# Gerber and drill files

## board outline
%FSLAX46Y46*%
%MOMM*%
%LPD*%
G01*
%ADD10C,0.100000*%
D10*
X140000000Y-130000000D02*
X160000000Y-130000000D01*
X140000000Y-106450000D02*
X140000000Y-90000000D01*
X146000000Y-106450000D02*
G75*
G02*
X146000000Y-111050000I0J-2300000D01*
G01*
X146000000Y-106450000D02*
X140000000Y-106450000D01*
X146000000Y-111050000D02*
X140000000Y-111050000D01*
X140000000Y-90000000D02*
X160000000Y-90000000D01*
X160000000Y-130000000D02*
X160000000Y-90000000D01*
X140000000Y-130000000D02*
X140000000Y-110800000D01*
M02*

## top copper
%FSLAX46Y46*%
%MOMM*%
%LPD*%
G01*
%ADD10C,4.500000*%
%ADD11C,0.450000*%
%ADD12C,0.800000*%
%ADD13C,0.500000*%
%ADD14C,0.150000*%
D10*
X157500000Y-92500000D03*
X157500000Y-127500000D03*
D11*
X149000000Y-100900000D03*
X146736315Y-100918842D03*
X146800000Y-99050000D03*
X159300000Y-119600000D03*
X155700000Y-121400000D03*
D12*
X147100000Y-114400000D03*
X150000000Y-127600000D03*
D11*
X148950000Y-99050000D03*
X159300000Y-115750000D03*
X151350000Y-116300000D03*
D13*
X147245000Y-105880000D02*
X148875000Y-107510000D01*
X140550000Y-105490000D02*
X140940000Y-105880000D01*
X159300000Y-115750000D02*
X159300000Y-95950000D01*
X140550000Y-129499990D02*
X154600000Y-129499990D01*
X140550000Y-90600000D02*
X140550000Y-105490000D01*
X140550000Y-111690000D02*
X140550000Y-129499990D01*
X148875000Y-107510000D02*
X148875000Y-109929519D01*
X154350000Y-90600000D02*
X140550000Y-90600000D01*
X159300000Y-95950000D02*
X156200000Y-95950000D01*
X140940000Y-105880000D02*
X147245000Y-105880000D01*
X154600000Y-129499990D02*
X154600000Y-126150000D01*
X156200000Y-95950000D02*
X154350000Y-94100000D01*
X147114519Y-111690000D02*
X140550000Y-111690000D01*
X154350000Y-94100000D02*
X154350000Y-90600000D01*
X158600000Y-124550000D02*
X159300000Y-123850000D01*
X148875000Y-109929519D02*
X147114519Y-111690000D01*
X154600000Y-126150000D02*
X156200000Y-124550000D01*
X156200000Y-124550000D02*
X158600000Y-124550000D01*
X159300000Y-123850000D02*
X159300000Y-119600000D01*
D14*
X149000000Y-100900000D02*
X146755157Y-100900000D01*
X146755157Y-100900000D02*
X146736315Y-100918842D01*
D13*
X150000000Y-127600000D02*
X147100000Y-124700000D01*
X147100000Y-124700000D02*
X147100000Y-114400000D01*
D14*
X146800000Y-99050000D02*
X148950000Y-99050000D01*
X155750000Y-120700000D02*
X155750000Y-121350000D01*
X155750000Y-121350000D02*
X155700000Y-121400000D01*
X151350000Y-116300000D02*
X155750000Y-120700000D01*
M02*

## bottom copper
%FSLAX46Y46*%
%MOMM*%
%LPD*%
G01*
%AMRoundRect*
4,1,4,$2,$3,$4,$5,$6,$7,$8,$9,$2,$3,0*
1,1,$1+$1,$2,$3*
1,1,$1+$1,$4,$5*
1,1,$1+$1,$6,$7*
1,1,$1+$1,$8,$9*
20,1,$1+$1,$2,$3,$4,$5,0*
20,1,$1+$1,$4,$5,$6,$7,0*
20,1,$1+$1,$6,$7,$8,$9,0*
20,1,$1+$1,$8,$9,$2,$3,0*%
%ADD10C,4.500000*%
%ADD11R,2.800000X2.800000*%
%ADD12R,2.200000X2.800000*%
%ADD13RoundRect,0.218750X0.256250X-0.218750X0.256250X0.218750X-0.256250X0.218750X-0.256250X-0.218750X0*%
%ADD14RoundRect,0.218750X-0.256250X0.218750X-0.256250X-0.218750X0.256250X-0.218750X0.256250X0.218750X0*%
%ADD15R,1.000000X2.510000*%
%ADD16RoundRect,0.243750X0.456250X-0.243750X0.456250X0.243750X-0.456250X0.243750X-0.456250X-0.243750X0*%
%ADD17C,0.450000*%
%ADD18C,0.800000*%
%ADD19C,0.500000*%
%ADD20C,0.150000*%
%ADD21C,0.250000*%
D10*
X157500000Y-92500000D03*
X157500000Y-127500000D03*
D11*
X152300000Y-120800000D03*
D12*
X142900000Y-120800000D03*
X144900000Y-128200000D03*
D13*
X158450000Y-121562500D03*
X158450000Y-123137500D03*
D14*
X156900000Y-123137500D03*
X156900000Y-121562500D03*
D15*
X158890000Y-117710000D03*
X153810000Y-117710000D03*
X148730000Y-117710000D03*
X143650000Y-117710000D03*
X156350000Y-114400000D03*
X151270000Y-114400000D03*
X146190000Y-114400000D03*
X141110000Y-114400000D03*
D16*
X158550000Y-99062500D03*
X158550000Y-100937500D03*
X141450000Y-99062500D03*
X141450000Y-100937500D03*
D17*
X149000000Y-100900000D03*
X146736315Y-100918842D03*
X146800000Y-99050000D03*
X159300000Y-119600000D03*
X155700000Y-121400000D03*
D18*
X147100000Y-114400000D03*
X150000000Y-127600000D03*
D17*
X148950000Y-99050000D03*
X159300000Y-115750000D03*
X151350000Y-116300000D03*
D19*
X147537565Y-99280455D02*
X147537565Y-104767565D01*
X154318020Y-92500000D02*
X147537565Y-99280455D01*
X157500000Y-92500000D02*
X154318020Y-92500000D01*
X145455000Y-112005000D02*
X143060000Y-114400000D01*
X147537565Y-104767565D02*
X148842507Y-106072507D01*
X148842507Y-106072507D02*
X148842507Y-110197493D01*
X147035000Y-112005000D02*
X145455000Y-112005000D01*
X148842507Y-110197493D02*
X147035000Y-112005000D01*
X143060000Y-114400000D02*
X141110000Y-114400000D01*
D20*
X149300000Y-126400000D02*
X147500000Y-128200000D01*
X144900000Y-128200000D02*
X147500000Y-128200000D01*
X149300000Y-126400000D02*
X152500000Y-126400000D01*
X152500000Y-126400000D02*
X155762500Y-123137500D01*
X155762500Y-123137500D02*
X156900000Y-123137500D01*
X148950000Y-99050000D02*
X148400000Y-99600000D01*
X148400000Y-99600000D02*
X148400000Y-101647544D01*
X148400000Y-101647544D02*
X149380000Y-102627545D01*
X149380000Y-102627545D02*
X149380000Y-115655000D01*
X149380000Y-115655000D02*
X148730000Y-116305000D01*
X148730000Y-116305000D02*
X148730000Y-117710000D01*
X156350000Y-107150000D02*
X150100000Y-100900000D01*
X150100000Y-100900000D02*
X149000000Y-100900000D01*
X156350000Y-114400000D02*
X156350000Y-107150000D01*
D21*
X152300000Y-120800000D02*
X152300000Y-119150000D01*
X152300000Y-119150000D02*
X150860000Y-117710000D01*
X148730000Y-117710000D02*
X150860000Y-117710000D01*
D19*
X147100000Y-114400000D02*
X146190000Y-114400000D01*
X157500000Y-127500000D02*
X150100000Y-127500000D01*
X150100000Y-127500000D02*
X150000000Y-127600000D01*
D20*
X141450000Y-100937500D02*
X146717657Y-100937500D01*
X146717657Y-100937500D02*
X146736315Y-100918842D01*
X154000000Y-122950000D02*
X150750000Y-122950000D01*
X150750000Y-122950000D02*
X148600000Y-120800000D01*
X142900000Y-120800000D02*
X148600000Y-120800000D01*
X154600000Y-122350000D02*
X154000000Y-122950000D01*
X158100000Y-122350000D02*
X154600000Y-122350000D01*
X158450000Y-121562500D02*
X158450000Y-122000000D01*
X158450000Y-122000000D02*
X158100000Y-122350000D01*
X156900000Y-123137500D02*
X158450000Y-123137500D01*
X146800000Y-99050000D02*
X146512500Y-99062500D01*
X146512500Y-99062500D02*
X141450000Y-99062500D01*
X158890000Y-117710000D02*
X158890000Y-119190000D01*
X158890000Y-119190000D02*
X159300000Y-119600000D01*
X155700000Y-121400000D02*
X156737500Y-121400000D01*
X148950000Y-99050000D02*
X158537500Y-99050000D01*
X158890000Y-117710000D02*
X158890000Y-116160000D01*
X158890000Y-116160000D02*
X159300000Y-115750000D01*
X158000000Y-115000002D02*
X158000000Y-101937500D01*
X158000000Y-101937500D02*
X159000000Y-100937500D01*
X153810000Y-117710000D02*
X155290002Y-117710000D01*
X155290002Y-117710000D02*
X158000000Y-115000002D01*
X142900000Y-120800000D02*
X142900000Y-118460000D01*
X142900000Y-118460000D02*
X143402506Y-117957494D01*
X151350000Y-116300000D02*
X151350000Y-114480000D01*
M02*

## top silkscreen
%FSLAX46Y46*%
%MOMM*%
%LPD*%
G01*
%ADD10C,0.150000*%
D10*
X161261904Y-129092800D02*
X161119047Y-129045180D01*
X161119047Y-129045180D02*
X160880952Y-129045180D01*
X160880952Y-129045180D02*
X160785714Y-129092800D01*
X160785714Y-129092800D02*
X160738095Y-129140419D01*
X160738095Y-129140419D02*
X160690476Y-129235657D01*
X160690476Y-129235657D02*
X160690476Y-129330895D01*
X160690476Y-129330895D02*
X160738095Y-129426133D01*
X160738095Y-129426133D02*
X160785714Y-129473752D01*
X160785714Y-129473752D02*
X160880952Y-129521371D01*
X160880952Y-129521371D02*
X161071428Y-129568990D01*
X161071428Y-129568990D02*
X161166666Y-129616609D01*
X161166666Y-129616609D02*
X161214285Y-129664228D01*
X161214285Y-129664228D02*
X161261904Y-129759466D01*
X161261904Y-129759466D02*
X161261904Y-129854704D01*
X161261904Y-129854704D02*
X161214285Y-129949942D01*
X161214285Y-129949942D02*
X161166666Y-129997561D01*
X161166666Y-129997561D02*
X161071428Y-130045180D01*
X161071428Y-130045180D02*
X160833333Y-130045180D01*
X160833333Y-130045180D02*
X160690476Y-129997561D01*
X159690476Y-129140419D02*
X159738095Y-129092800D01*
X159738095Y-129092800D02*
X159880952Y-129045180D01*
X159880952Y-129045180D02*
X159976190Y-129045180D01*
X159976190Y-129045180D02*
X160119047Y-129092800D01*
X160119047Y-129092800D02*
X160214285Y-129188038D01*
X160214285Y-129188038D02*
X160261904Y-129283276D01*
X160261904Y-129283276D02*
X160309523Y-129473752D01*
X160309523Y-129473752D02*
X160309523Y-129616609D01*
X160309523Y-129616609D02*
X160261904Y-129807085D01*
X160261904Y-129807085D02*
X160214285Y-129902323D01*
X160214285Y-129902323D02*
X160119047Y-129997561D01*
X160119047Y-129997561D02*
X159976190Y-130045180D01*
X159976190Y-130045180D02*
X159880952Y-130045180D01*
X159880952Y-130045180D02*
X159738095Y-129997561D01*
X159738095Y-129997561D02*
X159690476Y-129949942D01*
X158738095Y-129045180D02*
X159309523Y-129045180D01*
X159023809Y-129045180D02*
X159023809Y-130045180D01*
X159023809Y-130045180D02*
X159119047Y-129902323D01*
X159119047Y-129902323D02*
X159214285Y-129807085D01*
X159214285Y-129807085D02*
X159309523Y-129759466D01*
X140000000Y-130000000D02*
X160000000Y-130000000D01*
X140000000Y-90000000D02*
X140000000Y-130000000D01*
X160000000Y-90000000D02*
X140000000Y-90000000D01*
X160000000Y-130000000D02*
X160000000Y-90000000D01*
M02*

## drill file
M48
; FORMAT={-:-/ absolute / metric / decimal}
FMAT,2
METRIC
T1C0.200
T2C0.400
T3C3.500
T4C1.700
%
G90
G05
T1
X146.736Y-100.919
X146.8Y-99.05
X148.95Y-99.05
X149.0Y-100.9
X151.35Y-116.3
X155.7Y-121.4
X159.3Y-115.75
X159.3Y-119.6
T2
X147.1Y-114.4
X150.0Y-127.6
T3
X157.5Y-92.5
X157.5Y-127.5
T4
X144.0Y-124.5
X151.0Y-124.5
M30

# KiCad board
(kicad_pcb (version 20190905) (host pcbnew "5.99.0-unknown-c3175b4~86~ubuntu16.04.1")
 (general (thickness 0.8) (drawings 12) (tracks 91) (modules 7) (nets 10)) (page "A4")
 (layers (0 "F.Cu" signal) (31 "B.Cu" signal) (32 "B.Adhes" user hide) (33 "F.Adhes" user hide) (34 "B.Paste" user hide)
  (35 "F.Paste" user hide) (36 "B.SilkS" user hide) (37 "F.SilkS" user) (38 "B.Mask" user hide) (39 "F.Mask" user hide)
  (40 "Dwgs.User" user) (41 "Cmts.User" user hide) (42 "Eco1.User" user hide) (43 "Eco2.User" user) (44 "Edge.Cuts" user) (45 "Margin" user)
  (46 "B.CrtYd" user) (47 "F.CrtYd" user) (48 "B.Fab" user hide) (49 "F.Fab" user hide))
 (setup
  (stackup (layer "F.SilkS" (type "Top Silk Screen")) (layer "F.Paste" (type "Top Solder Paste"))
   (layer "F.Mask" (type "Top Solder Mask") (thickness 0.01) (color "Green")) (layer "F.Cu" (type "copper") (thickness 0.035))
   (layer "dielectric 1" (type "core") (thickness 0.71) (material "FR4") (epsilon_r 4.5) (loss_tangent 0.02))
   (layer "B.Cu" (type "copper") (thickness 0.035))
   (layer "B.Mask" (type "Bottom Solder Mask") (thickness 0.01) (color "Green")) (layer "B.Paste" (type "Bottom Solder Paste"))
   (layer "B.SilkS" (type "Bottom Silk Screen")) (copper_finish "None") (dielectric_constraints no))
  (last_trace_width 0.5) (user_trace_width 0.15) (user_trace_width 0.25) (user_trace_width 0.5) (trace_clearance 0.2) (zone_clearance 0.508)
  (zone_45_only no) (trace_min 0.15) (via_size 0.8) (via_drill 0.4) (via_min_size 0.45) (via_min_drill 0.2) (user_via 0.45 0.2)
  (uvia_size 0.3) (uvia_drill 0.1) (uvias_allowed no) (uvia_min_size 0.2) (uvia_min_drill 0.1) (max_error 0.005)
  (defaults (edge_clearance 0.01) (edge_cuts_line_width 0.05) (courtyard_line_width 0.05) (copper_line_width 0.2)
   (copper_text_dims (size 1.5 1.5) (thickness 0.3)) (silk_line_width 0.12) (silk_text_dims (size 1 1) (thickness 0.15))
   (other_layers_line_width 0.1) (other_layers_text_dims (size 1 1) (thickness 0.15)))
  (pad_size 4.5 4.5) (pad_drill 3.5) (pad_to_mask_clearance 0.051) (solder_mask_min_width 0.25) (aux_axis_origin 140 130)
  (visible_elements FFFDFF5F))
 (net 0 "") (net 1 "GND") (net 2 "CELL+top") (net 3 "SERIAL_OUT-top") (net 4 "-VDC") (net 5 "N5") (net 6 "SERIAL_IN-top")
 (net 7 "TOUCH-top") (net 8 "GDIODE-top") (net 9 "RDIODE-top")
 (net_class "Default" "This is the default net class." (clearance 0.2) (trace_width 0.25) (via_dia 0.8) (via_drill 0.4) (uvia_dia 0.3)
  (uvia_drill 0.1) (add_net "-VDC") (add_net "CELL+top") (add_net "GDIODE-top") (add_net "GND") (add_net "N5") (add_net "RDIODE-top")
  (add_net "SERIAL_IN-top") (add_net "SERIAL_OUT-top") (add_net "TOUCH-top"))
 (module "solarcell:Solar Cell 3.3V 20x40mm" (layer "F.Cu") (at 160 130 180)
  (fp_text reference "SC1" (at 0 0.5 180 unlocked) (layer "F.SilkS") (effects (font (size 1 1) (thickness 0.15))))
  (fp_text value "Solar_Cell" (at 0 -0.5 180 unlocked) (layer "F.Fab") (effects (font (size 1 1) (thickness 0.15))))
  (fp_line (start 20 0) (end 0 0) (layer "F.SilkS") (width 0.15))
  (fp_line (start 20 40) (end 20 0) (layer "F.SilkS") (width 0.15))
  (fp_line (start 0 40) (end 20 40) (layer "F.SilkS") (width 0.15))
  (fp_line (start 0 0) (end 0 40) (layer "F.SilkS") (width 0.15))
  (pad "2" thru_hole circle (at 2.5 37.5 180) (size 4.5 4.5) (drill 3.5) (layers *.Cu *.Mask) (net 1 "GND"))
  (pad "1" thru_hole circle (at 2.5 2.5 180) (size 4.5 4.5) (drill 3.5) (layers *.Cu *.Mask) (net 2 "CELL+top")))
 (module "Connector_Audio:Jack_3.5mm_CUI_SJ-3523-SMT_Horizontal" (layer "B.Cu") (at 146.5 124.5 -90)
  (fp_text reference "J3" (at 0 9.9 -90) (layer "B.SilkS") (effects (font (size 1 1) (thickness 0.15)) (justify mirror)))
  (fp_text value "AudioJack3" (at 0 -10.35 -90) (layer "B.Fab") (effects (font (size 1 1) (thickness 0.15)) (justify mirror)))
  (pad "" np_thru_hole circle (at 0 -4.5 270) (size 1.7 1.7) (drill 1.7) (layers *.Cu *.Mask))
  (pad "" np_thru_hole circle (at 0 2.5 270) (size 1.7 1.7) (drill 1.7) (layers *.Cu *.Mask))
  (pad "T" smd rect (at -3.7 -5.8 270) (size 2.8 2.8) (layers "B.Cu" "B.Paste" "B.Mask") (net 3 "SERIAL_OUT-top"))
  (pad "S" smd rect (at -3.7 3.6 270) (size 2.8 2.2) (layers "B.Cu" "B.Paste" "B.Mask") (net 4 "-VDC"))
  (pad "R" smd rect (at 3.7 1.6 270) (size 2.8 2.2) (layers "B.Cu" "B.Paste" "B.Mask") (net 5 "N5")))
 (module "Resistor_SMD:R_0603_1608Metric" (layer "B.Cu") (at 158.45 122.35 90)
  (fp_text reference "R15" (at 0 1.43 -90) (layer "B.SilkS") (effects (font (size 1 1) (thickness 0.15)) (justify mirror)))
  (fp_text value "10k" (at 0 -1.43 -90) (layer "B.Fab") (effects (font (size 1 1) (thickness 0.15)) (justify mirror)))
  (pad "2" smd roundrect (at 0.7875 0 90) (size 0.875 0.95) (layers "B.Cu" "B.Paste" "B.Mask") (roundrect_rratio 0.25) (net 4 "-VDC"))
  (pad "1" smd roundrect (at -0.7875 0 90) (size 0.875 0.95) (layers "B.Cu" "B.Paste" "B.Mask") (roundrect_rratio 0.25) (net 5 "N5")))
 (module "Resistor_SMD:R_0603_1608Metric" (layer "B.Cu") (at 156.9 122.35 -90)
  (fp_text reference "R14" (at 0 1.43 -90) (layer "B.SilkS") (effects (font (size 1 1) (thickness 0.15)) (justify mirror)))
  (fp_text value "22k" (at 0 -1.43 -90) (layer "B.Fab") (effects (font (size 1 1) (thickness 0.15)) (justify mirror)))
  (pad "2" smd roundrect (at 0.7875 0 270) (size 0.875 0.95) (layers "B.Cu" "B.Paste" "B.Mask") (roundrect_rratio 0.25) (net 5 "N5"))
  (pad "1" smd roundrect (at -0.7875 0 270) (size 0.875 0.95) (layers "B.Cu" "B.Paste" "B.Mask") (roundrect_rratio 0.25)
   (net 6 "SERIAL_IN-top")))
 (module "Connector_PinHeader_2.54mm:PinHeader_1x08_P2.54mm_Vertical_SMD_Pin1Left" (layer "B.Cu") (at 150 116.055 -90)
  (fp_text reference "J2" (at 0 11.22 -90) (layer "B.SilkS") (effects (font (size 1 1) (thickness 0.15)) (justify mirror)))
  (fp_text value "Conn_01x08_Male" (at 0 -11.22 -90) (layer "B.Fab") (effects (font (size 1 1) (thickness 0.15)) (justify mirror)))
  (pad "8" smd rect (at 1.655 -8.89 270) (size 2.51 1) (layers "B.Cu" "B.Paste" "B.Mask") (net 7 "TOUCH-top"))
  (pad "6" smd rect (at 1.655 -3.81 270) (size 2.51 1) (layers "B.Cu" "B.Paste" "B.Mask") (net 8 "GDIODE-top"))
  (pad "4" smd rect (at 1.655 1.27 270) (size 2.51 1) (layers "B.Cu" "B.Paste" "B.Mask") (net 3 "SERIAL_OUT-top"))
  (pad "2" smd rect (at 1.655 6.35 270) (size 2.51 1) (layers "B.Cu" "B.Paste" "B.Mask") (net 4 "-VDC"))
  (pad "7" smd rect (at -1.655 -6.35 270) (size 2.51 1) (layers "B.Cu" "B.Paste" "B.Mask") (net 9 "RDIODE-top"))
  (pad "5" smd rect (at -1.655 -1.27 270) (size 2.51 1) (layers "B.Cu" "B.Paste" "B.Mask") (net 6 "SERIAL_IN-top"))
  (pad "3" smd rect (at -1.655 3.81 270) (size 2.51 1) (layers "B.Cu" "B.Paste" "B.Mask") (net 2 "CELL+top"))
  (pad "1" smd rect (at -1.655 8.89 270) (size 2.51 1) (layers "B.Cu" "B.Paste" "B.Mask") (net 1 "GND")))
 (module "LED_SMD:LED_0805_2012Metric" (layer "B.Cu") (at 158.55 100 90)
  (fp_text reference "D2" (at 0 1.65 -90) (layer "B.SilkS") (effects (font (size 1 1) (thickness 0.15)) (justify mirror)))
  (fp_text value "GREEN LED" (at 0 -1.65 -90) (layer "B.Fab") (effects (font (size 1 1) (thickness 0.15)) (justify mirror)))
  (pad "2" smd roundrect (at 0.9375 0 90) (size 0.975 1.4) (layers "B.Cu" "B.Paste" "B.Mask") (roundrect_rratio 0.25)
   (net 3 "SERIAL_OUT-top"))
  (pad "1" smd roundrect (at -0.9375 0 90) (size 0.975 1.4) (layers "B.Cu" "B.Paste" "B.Mask") (roundrect_rratio 0.25) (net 8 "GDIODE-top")))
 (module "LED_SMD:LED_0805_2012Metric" (layer "B.Cu") (at 141.45 100 90)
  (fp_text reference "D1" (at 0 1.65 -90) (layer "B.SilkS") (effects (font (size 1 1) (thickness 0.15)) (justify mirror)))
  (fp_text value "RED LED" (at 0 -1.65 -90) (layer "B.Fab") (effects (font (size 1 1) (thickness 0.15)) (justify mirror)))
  (pad "2" smd roundrect (at 0.9375 0 90) (size 0.975 1.4) (layers "B.Cu" "B.Paste" "B.Mask") (roundrect_rratio 0.25)
   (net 3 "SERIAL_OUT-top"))
  (pad "1" smd roundrect (at -0.9375 0 90) (size 0.975 1.4) (layers "B.Cu" "B.Paste" "B.Mask") (roundrect_rratio 0.25) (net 9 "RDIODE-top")))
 (gr_line (start 140 130) (end 160 130) (layer "Edge.Cuts") (width 0.1))
 (gr_line (start 140 106.45) (end 140 90) (layer "Edge.Cuts") (width 0.1))
 (gr_arc (start 146 108.75) (end 146 106.45) (angle 180) (layer "Edge.Cuts") (width 0.1))
 (gr_line (start 146 106.45) (end 140 106.45) (layer "Edge.Cuts") (width 0.1))
 (gr_line (start 146 111.05) (end 140 111.05) (layer "Edge.Cuts") (width 0.1))
 (gr_line (start 140 90) (end 160 90) (layer "Edge.Cuts") (width 0.1))
 (gr_line (start 160 130) (end 160 90) (layer "Edge.Cuts") (width 0.1))
 (gr_line (start 140 130) (end 140 110.8) (layer "Edge.Cuts") (width 0.1))
 (segment (start 147.537565 99.280455) (end 147.537565 104.767565) (width 0.5) (layer "B.Cu") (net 1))
 (segment (start 154.31802 92.5) (end 147.537565 99.280455) (width 0.5) (layer "B.Cu") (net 1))
 (segment (start 157.5 92.5) (end 154.31802 92.5) (width 0.5) (layer "B.Cu") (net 1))
 (segment (start 145.455 112.005) (end 143.06 114.4) (width 0.5) (layer "B.Cu") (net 1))
 (segment (start 147.537565 104.767565) (end 148.842507 106.072507) (width 0.5) (layer "B.Cu") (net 1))
 (segment (start 148.842507 106.072507) (end 148.842507 110.197493) (width 0.5) (layer "B.Cu") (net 1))
 (segment (start 147.035 112.005) (end 145.455 112.005) (width 0.5) (layer "B.Cu") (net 1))
 (segment (start 148.842507 110.197493) (end 147.035 112.005) (width 0.5) (layer "B.Cu") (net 1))
 (segment (start 143.06 114.4) (end 141.11 114.4) (width 0.5) (layer "B.Cu") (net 1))
 (segment (start 147.245 105.88) (end 148.875 107.51) (width 0.5) (layer "F.Cu") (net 7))
 (segment (start 140.55 105.49) (end 140.94 105.88) (width 0.5) (layer "F.Cu") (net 7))
 (segment (start 159.3 115.75) (end 159.3 95.95) (width 0.5) (layer "F.Cu") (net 7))
 (segment (start 140.55 129.49999) (end 154.6 129.49999) (width 0.5) (layer "F.Cu") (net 7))
 (segment (start 140.55 90.6) (end 140.55 105.49) (width 0.5) (layer "F.Cu") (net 7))
 (segment (start 140.55 111.69) (end 140.55 129.49999) (width 0.5) (layer "F.Cu") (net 7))
 (segment (start 148.875 107.51) (end 148.875 109.929519) (width 0.5) (layer "F.Cu") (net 7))
 (segment (start 154.35 90.6) (end 140.55 90.6) (width 0.5) (layer "F.Cu") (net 7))
 (segment (start 159.3 95.95) (end 156.2 95.95) (width 0.5) (layer "F.Cu") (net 7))
 (segment (start 140.94 105.88) (end 147.245 105.88) (width 0.5) (layer "F.Cu") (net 7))
 (segment (start 154.6 129.49999) (end 154.6 126.15) (width 0.5) (layer "F.Cu") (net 7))
 (segment (start 156.2 95.95) (end 154.35 94.1) (width 0.5) (layer "F.Cu") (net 7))
 (segment (start 147.114519 111.69) (end 140.55 111.69) (width 0.5) (layer "F.Cu") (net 7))
 (segment (start 154.35 94.1) (end 154.35 90.6) (width 0.5) (layer "F.Cu") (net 7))
 (segment (start 158.6 124.55) (end 159.3 123.85) (width 0.5) (layer "F.Cu") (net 7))
 (segment (start 148.875 109.929519) (end 147.114519 111.69) (width 0.5) (layer "F.Cu") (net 7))
 (segment (start 154.6 126.15) (end 156.2 124.55) (width 0.5) (layer "F.Cu") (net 7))
 (segment (start 156.2 124.55) (end 158.6 124.55) (width 0.5) (layer "F.Cu") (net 7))
 (segment (start 159.3 123.85) (end 159.3 119.6) (width 0.5) (layer "F.Cu") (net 7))
 (segment (start 149.3 126.4) (end 147.5 128.2) (width 0.15) (layer "B.Cu") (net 5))
 (segment (start 144.9 128.2) (end 147.5 128.2) (width 0.15) (layer "B.Cu") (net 5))
 (segment (start 149.3 126.4) (end 152.5 126.4) (width 0.15) (layer "B.Cu") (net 5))
 (segment (start 152.5 126.4) (end 155.7625 123.1375) (width 0.15) (layer "B.Cu") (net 5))
 (segment (start 155.7625 123.1375) (end 156.9 123.1375) (width 0.15) (layer "B.Cu") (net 5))
 (segment (start 148.95 99.05) (end 148.4 99.6) (width 0.15) (layer "B.Cu") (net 3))
 (segment (start 148.4 99.6) (end 148.4 101.647544) (width 0.15) (layer "B.Cu") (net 3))
 (segment (start 148.4 101.647544) (end 149.38 102.627545) (width 0.15) (layer "B.Cu") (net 3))
 (segment (start 149.38 102.627545) (end 149.38 115.655) (width 0.15) (layer "B.Cu") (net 3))
 (segment (start 149.38 115.655) (end 148.73 116.305) (width 0.15) (layer "B.Cu") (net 3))
 (segment (start 148.73 116.305) (end 148.73 117.71) (width 0.15) (layer "B.Cu") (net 3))
 (segment (start 149 100.9) (end 146.755157 100.9) (width 0.15) (layer "F.Cu") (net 9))
 (segment (start 146.755157 100.9) (end 146.736315 100.918842) (width 0.15) (layer "F.Cu") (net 9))
 (segment (start 156.35 107.15) (end 150.1 100.9) (width 0.15) (layer "B.Cu") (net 9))
 (via (at 149 100.9) (size 0.45) (drill 0.2) (layers "F.Cu" "B.Cu") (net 9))
 (segment (start 150.1 100.9) (end 149 100.9) (width 0.15) (layer "B.Cu") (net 9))
 (segment (start 156.35 114.4) (end 156.35 107.15) (width 0.15) (layer "B.Cu") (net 9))
 (segment (start 152.3 120.8) (end 152.3 119.15) (width 0.25) (layer "B.Cu") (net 3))
 (segment (start 152.3 119.15) (end 150.86 117.71) (width 0.25) (layer "B.Cu") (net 3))
 (segment (start 148.73 117.71) (end 150.86 117.71) (width 0.25) (layer "B.Cu") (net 3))
 (segment (start 147.1 114.4) (end 146.19 114.4) (width 0.5) (layer "B.Cu") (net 2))
 (segment (start 150 127.6) (end 147.1 124.7) (width 0.5) (layer "F.Cu") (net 2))
 (segment (start 147.1 124.7) (end 147.1 114.4) (width 0.5) (layer "F.Cu") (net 2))
 (segment (start 157.5 127.5) (end 150.1 127.5) (width 0.5) (layer "B.Cu") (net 2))
 (segment (start 150.1 127.5) (end 150 127.6) (width 0.5) (layer "B.Cu") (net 2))
 (segment (start 141.45 100.9375) (end 146.717657 100.9375) (width 0.15) (layer "B.Cu") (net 9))
 (segment (start 146.717657 100.9375) (end 146.736315 100.918842) (width 0.15) (layer "B.Cu") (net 9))
 (via (at 146.736315 100.918842) (size 0.45) (drill 0.2) (layers "F.Cu" "B.Cu") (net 9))
 (segment (start 154 122.95) (end 150.75 122.95) (width 0.15) (layer "B.Cu") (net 4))
 (segment (start 150.75 122.95) (end 148.6 120.8) (width 0.15) (layer "B.Cu") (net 4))
 (segment (start 142.9 120.8) (end 148.6 120.8) (width 0.15) (layer "B.Cu") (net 4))
 (segment (start 154.6 122.35) (end 154 122.95) (width 0.15) (layer "B.Cu") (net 4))
 (segment (start 158.1 122.35) (end 154.6 122.35) (width 0.15) (layer "B.Cu") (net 4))
 (segment (start 158.45 121.5625) (end 158.45 122) (width 0.15) (layer "B.Cu") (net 4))
 (segment (start 158.45 122) (end 158.1 122.35) (width 0.15) (layer "B.Cu") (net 4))
 (segment (start 156.9 123.1375) (end 158.45 123.1375) (width 0.15) (layer "B.Cu") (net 5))
 (segment (start 146.8 99.05) (end 146.5125 99.0625) (width 0.15) (layer "B.Cu") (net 3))
 (via (at 146.8 99.05) (size 0.45) (drill 0.2) (layers "F.Cu" "B.Cu") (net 3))
 (segment (start 146.5125 99.0625) (end 141.45 99.0625) (width 0.15) (layer "B.Cu") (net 3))
 (segment (start 146.8 99.05) (end 148.95 99.05) (width 0.15) (layer "F.Cu") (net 3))
 (segment (start 158.89 117.71) (end 158.89 119.19) (width 0.15) (layer "B.Cu") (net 7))
 (segment (start 158.89 119.19) (end 159.3 119.6) (width 0.15) (layer "B.Cu") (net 7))
 (via (at 159.3 119.6) (size 0.45) (drill 0.2) (layers "F.Cu" "B.Cu") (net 7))
 (segment (start 155.7 121.4) (end 156.7375 121.4) (width 0.15) (layer "B.Cu") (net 6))
 (segment (start 155.75 120.7) (end 155.75 121.35) (width 0.15) (layer "F.Cu") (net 6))
 (segment (start 155.75 121.35) (end 155.7 121.4) (width 0.15) (layer "F.Cu") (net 6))
 (via (at 155.7 121.4) (size 0.45) (drill 0.2) (layers "F.Cu" "B.Cu") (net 6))
 (segment (start 151.35 116.3) (end 155.75 120.7) (width 0.15) (layer "F.Cu") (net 6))
 (via (at 147.1 114.4) (size 0.8) (drill 0.4) (layers "F.Cu" "B.Cu") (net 2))
 (via (at 150 127.6) (size 0.8) (drill 0.4) (layers "F.Cu" "B.Cu") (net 2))
 (segment (start 148.95 99.05) (end 158.5375 99.05) (width 0.15) (layer "B.Cu") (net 3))
 (via (at 148.95 99.05) (size 0.45) (drill 0.2) (layers "F.Cu" "B.Cu") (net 3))
 (segment (start 158.89 117.71) (end 158.89 116.16) (width 0.15) (layer "B.Cu") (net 7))
 (segment (start 158.89 116.16) (end 159.3 115.75) (width 0.15) (layer "B.Cu") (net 7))
 (via (at 159.3 115.75) (size 0.45) (drill 0.2) (layers "F.Cu" "B.Cu") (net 7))
 (segment (start 158 115.000002) (end 158 101.9375) (width 0.15) (layer "B.Cu") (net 8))
 (segment (start 158 101.9375) (end 159 100.9375) (width 0.15) (layer "B.Cu") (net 8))
 (segment (start 153.81 117.71) (end 155.290002 117.71) (width 0.15) (layer "B.Cu") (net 8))
 (segment (start 155.290002 117.71) (end 158 115.000002) (width 0.15) (layer "B.Cu") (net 8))
 (segment (start 142.9 120.8) (end 142.9 118.46) (width 0.15) (layer "B.Cu") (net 4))
 (segment (start 142.9 118.46) (end 143.402506 117.957494) (width 0.15) (layer "B.Cu") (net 4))
 (segment (start 151.35 116.3) (end 151.35 114.48) (width 0.15) (layer "B.Cu") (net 6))
 (via (at 151.35 116.3) (size 0.45) (drill 0.2) (layers "F.Cu" "B.Cu") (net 6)))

